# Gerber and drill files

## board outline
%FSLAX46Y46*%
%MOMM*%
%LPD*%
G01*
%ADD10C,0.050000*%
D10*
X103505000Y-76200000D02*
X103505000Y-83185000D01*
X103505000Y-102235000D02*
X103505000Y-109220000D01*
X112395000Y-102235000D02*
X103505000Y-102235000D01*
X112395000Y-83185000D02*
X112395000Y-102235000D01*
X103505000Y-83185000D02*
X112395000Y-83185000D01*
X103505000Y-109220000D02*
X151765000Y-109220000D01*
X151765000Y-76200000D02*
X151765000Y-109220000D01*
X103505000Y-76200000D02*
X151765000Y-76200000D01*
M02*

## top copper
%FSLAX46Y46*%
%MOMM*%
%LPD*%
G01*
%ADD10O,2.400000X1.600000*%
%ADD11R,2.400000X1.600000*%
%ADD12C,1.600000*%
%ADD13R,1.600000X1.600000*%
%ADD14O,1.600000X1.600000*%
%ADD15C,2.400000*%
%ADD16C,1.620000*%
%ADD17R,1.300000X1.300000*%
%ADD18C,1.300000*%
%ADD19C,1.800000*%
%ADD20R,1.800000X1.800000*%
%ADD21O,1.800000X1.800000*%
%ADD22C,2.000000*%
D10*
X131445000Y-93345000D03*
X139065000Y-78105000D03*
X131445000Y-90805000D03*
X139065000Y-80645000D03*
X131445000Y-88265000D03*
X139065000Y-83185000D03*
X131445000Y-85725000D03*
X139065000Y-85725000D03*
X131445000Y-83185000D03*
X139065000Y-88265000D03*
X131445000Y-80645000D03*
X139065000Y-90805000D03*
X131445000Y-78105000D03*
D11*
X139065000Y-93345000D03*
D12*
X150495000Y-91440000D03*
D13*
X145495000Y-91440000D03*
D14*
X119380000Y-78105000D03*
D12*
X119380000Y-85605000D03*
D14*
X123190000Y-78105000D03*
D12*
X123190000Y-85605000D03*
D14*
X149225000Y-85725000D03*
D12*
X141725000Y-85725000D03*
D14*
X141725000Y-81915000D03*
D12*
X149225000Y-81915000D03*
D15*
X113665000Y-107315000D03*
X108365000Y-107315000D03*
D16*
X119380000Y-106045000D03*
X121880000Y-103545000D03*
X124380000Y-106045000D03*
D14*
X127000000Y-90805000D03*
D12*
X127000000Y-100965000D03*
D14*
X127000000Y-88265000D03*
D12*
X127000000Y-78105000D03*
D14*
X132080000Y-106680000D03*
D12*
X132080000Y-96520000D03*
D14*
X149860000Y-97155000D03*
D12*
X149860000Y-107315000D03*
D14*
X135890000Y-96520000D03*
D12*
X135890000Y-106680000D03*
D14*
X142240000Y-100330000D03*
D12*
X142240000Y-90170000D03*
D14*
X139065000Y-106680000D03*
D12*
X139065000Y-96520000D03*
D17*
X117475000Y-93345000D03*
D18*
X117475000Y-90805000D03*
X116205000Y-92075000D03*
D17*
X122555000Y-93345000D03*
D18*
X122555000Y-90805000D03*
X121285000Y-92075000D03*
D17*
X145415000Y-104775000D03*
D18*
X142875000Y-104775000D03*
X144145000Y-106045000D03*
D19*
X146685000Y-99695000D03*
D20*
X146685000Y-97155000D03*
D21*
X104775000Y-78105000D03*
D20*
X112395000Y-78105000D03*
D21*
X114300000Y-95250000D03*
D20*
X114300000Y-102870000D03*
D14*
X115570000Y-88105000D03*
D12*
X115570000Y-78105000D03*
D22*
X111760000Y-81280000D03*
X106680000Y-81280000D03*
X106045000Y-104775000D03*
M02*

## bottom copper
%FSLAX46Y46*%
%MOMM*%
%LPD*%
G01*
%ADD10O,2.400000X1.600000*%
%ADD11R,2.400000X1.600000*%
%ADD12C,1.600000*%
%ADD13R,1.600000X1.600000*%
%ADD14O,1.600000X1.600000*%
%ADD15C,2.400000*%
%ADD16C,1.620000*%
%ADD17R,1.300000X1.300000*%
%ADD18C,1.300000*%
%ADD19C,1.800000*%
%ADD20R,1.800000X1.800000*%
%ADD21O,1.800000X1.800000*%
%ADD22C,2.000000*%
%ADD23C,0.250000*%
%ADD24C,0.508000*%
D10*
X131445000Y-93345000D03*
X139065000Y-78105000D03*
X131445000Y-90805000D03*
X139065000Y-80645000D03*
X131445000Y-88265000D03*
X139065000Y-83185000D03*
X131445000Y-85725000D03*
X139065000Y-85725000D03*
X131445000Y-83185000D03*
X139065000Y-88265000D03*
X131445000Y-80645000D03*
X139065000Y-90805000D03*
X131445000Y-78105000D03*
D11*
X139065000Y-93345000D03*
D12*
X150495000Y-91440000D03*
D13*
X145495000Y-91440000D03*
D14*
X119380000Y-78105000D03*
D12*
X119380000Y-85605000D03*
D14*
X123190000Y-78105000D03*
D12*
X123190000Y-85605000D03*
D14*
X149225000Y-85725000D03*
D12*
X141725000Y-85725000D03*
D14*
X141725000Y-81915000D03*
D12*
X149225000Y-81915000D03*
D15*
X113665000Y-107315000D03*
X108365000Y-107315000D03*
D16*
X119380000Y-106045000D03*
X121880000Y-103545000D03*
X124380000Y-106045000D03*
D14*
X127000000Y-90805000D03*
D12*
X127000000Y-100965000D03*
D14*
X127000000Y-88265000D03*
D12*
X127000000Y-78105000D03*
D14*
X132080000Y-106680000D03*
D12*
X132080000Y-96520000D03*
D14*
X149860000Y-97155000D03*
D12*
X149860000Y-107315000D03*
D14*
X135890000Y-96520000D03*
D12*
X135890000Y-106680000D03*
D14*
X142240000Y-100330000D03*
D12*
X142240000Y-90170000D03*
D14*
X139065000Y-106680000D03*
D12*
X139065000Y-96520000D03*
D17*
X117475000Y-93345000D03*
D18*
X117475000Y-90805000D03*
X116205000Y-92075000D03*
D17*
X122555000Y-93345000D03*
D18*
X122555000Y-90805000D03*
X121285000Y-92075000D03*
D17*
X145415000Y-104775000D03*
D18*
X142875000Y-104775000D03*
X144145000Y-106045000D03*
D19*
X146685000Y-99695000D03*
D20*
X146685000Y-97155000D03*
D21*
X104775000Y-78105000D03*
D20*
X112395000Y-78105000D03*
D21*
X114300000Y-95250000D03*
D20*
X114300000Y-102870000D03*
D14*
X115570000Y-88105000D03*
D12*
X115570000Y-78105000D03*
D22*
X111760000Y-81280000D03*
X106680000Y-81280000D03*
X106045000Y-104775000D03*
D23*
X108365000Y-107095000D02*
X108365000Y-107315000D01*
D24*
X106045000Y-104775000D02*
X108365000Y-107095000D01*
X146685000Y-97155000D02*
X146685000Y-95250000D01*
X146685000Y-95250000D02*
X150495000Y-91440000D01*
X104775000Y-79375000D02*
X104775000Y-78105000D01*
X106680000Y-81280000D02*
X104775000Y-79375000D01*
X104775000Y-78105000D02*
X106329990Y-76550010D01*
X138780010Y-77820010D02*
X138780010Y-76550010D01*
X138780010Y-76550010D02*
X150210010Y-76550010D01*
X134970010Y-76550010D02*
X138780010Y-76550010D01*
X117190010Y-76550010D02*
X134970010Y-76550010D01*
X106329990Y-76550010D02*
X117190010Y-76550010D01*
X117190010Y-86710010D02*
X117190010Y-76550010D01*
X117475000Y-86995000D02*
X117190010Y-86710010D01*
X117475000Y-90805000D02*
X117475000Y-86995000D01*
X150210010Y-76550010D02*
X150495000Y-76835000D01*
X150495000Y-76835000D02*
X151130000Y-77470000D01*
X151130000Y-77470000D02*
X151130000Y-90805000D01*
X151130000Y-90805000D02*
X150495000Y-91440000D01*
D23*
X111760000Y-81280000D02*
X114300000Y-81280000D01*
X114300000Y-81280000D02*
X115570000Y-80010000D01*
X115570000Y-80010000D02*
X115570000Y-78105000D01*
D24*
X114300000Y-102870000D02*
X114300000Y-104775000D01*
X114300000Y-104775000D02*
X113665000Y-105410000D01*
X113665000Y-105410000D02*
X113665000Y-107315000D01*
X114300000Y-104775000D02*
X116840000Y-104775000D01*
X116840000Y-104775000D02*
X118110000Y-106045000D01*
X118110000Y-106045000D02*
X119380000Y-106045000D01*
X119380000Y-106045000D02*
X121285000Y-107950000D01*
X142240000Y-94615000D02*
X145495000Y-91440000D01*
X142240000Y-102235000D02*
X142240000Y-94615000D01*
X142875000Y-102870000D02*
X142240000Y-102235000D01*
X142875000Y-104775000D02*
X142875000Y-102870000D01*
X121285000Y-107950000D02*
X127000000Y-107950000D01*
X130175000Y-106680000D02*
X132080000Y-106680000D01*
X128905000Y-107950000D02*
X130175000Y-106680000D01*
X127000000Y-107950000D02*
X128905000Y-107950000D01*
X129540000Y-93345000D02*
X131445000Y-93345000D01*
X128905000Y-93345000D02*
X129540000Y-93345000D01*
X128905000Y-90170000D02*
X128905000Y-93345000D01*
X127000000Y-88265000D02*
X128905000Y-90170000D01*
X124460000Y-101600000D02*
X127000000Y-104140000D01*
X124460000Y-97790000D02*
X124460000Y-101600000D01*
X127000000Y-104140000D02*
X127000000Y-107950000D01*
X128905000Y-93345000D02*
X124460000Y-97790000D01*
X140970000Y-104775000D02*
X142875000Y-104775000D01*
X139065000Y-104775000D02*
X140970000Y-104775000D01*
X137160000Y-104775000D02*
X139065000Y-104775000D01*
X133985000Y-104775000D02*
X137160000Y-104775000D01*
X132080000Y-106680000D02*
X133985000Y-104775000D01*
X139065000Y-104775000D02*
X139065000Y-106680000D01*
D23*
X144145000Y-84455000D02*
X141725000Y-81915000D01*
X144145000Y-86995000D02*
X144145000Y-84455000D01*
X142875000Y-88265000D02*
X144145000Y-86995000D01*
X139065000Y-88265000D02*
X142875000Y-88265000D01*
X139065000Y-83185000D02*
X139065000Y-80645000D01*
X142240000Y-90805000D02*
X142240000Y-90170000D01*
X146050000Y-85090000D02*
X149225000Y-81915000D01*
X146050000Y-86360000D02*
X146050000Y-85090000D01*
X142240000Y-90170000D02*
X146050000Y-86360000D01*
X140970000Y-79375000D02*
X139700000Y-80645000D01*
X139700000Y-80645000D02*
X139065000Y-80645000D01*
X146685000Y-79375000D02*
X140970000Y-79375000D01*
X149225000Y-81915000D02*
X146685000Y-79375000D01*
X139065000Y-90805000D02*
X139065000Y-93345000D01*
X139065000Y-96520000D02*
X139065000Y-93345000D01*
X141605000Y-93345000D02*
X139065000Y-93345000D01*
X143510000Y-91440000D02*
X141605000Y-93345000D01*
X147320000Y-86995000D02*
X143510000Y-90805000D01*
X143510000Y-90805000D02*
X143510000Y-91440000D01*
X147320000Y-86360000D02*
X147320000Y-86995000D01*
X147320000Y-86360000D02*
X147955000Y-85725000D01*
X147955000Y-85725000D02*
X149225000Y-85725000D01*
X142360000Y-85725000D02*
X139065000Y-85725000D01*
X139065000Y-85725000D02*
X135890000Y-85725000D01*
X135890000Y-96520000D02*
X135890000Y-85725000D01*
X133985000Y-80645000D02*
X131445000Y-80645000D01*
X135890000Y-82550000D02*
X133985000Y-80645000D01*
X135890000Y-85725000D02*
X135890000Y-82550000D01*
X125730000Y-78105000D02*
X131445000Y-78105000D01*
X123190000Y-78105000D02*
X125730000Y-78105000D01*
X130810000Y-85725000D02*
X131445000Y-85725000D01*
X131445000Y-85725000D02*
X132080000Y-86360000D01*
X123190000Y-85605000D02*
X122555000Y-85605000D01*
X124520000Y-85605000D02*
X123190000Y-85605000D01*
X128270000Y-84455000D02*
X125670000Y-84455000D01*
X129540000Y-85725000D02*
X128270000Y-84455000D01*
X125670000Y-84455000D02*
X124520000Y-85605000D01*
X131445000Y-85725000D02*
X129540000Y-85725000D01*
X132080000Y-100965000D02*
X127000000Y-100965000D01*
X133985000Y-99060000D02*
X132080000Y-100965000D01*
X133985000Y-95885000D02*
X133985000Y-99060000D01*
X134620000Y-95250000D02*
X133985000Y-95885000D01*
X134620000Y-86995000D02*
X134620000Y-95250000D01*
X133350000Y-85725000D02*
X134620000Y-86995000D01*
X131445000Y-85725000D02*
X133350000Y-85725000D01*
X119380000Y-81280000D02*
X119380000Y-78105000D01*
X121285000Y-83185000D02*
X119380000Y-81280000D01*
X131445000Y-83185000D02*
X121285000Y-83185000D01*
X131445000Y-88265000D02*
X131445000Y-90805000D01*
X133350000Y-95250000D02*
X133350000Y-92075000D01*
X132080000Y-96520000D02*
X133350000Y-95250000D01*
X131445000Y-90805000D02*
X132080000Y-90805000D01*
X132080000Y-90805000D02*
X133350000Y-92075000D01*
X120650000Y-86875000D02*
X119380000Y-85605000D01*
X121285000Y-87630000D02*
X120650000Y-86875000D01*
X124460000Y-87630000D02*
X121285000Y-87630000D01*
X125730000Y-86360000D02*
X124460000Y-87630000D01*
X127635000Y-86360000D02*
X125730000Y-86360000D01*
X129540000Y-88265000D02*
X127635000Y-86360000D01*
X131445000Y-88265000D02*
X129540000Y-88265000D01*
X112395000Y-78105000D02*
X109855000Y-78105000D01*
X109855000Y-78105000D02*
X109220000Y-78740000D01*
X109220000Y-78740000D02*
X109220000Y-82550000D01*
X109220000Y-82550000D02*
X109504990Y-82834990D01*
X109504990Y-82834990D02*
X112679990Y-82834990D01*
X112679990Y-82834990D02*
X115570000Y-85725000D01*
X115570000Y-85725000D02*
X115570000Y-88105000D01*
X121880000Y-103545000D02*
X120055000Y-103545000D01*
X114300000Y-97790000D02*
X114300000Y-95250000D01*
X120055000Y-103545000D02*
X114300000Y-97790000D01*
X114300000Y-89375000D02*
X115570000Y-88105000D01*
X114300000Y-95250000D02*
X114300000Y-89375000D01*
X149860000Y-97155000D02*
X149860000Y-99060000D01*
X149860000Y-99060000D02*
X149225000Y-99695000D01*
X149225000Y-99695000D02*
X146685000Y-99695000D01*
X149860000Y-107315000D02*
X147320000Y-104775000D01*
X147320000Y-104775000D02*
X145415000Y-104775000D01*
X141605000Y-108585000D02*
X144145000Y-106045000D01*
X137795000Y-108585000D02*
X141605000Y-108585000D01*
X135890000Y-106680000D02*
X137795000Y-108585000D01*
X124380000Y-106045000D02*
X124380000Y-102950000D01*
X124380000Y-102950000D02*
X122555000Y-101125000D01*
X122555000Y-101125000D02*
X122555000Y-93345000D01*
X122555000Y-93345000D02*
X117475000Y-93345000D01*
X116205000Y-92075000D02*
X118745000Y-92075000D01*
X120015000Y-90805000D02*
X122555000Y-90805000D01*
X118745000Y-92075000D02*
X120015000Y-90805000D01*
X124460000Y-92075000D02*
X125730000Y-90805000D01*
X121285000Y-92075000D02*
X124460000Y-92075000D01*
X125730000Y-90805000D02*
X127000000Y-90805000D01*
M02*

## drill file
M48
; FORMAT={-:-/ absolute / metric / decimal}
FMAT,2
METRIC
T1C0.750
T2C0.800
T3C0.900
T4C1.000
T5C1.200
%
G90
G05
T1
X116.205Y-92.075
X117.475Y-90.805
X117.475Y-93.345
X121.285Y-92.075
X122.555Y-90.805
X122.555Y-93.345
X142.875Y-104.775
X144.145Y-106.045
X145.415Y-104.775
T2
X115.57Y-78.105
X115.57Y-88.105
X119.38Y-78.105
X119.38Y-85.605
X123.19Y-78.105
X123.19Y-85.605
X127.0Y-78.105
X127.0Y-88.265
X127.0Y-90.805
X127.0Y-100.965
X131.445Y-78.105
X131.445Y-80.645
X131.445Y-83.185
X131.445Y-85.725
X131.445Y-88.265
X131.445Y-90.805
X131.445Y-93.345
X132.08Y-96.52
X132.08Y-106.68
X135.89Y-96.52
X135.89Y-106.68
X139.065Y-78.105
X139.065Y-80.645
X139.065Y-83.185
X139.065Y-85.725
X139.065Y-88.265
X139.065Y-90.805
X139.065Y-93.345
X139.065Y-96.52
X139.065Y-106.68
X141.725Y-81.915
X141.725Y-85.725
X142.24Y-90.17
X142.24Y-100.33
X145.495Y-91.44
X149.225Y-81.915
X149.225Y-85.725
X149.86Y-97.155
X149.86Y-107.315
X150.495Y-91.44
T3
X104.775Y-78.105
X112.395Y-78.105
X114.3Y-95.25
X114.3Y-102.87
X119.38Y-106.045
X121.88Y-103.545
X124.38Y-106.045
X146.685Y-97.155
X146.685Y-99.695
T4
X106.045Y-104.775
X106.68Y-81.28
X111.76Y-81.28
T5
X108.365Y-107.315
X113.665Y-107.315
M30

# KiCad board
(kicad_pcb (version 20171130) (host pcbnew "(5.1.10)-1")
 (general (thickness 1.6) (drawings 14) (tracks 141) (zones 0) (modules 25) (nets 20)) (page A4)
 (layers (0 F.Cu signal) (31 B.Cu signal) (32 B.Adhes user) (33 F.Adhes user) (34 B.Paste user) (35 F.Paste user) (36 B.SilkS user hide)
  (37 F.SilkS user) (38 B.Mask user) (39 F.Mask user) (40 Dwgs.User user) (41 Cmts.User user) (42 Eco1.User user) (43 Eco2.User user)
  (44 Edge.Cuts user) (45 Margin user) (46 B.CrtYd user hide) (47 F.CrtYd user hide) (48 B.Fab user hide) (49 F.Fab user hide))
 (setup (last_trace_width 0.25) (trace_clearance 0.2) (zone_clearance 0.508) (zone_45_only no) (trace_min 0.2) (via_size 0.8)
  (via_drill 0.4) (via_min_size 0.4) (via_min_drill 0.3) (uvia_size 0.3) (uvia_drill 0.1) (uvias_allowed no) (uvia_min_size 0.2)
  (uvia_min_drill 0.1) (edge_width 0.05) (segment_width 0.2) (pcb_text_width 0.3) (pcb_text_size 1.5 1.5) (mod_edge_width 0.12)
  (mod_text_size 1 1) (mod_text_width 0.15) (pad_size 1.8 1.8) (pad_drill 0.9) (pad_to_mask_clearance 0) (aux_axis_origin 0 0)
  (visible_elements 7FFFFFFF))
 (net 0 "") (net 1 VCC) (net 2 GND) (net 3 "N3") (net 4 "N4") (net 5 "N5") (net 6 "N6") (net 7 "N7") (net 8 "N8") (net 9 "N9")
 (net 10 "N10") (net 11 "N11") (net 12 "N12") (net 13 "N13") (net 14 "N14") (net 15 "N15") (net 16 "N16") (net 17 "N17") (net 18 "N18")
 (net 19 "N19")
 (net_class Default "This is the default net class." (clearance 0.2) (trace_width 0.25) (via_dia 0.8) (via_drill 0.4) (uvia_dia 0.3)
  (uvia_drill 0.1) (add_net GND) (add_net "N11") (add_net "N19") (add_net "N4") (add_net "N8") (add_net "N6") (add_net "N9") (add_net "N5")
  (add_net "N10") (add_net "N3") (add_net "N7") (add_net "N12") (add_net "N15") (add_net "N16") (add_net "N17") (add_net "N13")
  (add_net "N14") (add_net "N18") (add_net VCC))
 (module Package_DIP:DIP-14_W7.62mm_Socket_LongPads (layer F.Cu) (at 139.065 93.345 180)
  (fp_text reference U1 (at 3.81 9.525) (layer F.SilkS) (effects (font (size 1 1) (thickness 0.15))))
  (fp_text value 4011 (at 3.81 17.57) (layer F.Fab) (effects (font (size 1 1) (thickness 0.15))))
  (pad 14 thru_hole oval (at 7.62 0 180) (size 2.4 1.6) (drill 0.8) (layers *.Cu *.Mask) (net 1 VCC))
  (pad 7 thru_hole oval (at 0 15.24 180) (size 2.4 1.6) (drill 0.8) (layers *.Cu *.Mask) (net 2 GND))
  (pad 13 thru_hole oval (at 7.62 2.54 180) (size 2.4 1.6) (drill 0.8) (layers *.Cu *.Mask) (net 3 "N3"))
  (pad 6 thru_hole oval (at 0 12.7 180) (size 2.4 1.6) (drill 0.8) (layers *.Cu *.Mask) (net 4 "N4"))
  (pad 12 thru_hole oval (at 7.62 5.08 180) (size 2.4 1.6) (drill 0.8) (layers *.Cu *.Mask) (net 3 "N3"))
  (pad 5 thru_hole oval (at 0 10.16 180) (size 2.4 1.6) (drill 0.8) (layers *.Cu *.Mask) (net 4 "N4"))
  (pad 11 thru_hole oval (at 7.62 7.62 180) (size 2.4 1.6) (drill 0.8) (layers *.Cu *.Mask) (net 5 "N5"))
  (pad 4 thru_hole oval (at 0 7.62 180) (size 2.4 1.6) (drill 0.8) (layers *.Cu *.Mask) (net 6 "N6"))
  (pad 10 thru_hole oval (at 7.62 10.16 180) (size 2.4 1.6) (drill 0.8) (layers *.Cu *.Mask) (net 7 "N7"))
  (pad 3 thru_hole oval (at 0 5.08 180) (size 2.4 1.6) (drill 0.8) (layers *.Cu *.Mask) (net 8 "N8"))
  (pad 9 thru_hole oval (at 7.62 12.7 180) (size 2.4 1.6) (drill 0.8) (layers *.Cu *.Mask) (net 6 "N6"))
  (pad 2 thru_hole oval (at 0 2.54 180) (size 2.4 1.6) (drill 0.8) (layers *.Cu *.Mask) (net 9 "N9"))
  (pad 8 thru_hole oval (at 7.62 15.24 180) (size 2.4 1.6) (drill 0.8) (layers *.Cu *.Mask) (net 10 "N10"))
  (pad 1 thru_hole rect (at 0 0 180) (size 2.4 1.6) (drill 0.8) (layers *.Cu *.Mask) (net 9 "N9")))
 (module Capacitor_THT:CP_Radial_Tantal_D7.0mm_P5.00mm (layer F.Cu) (at 145.495 91.44)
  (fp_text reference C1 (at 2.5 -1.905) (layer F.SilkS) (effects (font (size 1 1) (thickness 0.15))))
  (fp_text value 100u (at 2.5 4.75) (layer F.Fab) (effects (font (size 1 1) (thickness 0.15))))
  (pad 2 thru_hole circle (at 5 0) (size 1.6 1.6) (drill 0.8) (layers *.Cu *.Mask) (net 2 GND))
  (pad 1 thru_hole rect (at 0 0) (size 1.6 1.6) (drill 0.8) (layers *.Cu *.Mask) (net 1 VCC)))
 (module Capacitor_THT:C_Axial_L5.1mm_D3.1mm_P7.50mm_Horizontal (layer F.Cu) (at 119.38 85.605 90)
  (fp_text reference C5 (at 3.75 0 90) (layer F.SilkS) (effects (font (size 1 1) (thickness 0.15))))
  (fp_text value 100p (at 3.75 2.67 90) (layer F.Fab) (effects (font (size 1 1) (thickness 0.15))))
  (pad 2 thru_hole oval (at 7.5 0 90) (size 1.6 1.6) (drill 0.8) (layers *.Cu *.Mask) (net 7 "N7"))
  (pad 1 thru_hole circle (at 0 0 90) (size 1.6 1.6) (drill 0.8) (layers *.Cu *.Mask) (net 3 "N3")))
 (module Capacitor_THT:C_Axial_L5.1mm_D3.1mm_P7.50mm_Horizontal (layer F.Cu) (at 123.19 85.605 90)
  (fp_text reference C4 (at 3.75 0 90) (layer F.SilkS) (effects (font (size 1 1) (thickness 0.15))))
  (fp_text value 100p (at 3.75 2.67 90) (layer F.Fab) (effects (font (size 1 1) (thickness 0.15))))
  (pad 2 thru_hole oval (at 7.5 0 90) (size 1.6 1.6) (drill 0.8) (layers *.Cu *.Mask) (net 10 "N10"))
  (pad 1 thru_hole circle (at 0 0 90) (size 1.6 1.6) (drill 0.8) (layers *.Cu *.Mask) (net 5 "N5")))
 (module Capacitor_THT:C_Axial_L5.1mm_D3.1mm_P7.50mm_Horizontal (layer F.Cu) (at 141.725 85.725)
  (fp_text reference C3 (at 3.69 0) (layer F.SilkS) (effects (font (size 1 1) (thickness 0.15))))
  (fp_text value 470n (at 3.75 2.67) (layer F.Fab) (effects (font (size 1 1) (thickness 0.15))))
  (pad 2 thru_hole oval (at 7.5 0) (size 1.6 1.6) (drill 0.8) (layers *.Cu *.Mask) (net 9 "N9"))
  (pad 1 thru_hole circle (at 0 0) (size 1.6 1.6) (drill 0.8) (layers *.Cu *.Mask) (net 6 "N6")))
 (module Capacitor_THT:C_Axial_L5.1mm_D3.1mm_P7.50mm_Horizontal (layer F.Cu) (at 149.225 81.915 180)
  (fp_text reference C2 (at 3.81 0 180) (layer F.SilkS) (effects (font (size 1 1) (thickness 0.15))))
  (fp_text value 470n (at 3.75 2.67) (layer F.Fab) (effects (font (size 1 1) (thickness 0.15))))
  (pad 2 thru_hole oval (at 7.5 0 180) (size 1.6 1.6) (drill 0.8) (layers *.Cu *.Mask) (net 8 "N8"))
  (pad 1 thru_hole circle (at 0 0 180) (size 1.6 1.6) (drill 0.8) (layers *.Cu *.Mask) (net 4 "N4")))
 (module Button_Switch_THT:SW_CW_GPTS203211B (layer B.Cu) (at 108.365 107.315 270)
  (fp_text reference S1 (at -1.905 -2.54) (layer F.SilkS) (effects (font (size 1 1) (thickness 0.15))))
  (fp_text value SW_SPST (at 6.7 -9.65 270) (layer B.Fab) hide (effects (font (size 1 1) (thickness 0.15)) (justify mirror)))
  (pad 2 thru_hole circle (at 0 -5.3 270) (size 2.4 2.4) (drill 1.2) (layers *.Cu *.Mask) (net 1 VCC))
  (pad 1 thru_hole circle (at 0 0 270) (size 2.4 2.4) (drill 1.2) (layers *.Cu *.Mask) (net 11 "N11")))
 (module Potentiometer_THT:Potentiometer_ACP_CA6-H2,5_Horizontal (layer F.Cu) (at 119.38 106.045 90)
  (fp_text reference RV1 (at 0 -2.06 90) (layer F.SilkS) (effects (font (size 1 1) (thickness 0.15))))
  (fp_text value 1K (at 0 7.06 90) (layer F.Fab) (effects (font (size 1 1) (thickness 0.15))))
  (pad 1 thru_hole circle (at 0 0 90) (size 1.62 1.62) (drill 0.9) (layers *.Cu *.Mask) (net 1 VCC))
  (pad 2 thru_hole circle (at 2.5 2.5 90) (size 1.62 1.62) (drill 0.9) (layers *.Cu *.Mask) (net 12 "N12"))
  (pad 3 thru_hole circle (at 0 5 90) (size 1.62 1.62) (drill 0.9) (layers *.Cu *.Mask) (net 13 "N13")))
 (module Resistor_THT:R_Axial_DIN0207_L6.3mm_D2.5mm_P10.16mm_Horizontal (layer F.Cu) (at 127 100.965 90)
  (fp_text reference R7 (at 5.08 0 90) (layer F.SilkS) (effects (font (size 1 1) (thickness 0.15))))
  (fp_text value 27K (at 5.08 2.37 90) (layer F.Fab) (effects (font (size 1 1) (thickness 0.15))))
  (pad 2 thru_hole oval (at 10.16 0 90) (size 1.6 1.6) (drill 0.8) (layers *.Cu *.Mask) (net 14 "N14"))
  (pad 1 thru_hole circle (at 0 0 90) (size 1.6 1.6) (drill 0.8) (layers *.Cu *.Mask) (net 5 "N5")))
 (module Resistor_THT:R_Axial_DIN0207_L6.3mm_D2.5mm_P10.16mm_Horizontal (layer F.Cu) (at 127 78.105 270)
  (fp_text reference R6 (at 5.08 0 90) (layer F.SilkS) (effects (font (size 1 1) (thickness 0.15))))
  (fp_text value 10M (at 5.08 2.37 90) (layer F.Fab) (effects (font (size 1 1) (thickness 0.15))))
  (pad 2 thru_hole oval (at 10.16 0 270) (size 1.6 1.6) (drill 0.8) (layers *.Cu *.Mask) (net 1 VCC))
  (pad 1 thru_hole circle (at 0 0 270) (size 1.6 1.6) (drill 0.8) (layers *.Cu *.Mask) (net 10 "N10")))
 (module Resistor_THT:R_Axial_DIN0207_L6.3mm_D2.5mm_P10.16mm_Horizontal (layer F.Cu) (at 132.08 96.52 270)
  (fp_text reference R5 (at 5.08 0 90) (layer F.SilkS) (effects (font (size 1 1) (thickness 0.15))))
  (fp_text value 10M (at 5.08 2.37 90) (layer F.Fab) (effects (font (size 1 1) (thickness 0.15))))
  (pad 2 thru_hole oval (at 10.16 0 270) (size 1.6 1.6) (drill 0.8) (layers *.Cu *.Mask) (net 1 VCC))
  (pad 1 thru_hole circle (at 0 0 270) (size 1.6 1.6) (drill 0.8) (layers *.Cu *.Mask) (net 3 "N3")))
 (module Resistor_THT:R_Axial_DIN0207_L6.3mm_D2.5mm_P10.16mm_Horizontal (layer F.Cu) (at 149.86 107.315 90)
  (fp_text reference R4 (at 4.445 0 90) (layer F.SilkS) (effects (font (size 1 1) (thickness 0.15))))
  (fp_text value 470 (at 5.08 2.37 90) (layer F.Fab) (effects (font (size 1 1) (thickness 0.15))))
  (pad 2 thru_hole oval (at 10.16 0 90) (size 1.6 1.6) (drill 0.8) (layers *.Cu *.Mask) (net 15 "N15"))
  (pad 1 thru_hole circle (at 0 0 90) (size 1.6 1.6) (drill 0.8) (layers *.Cu *.Mask) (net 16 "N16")))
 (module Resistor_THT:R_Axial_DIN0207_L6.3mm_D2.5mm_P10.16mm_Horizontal (layer F.Cu) (at 135.89 106.68 90)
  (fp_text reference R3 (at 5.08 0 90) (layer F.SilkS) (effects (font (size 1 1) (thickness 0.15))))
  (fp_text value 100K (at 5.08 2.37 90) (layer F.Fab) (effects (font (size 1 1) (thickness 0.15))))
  (pad 2 thru_hole oval (at 10.16 0 90) (size 1.6 1.6) (drill 0.8) (layers *.Cu *.Mask) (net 6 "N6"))
  (pad 1 thru_hole circle (at 0 0 90) (size 1.6 1.6) (drill 0.8) (layers *.Cu *.Mask) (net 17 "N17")))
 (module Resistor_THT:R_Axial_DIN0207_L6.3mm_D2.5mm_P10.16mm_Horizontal (layer F.Cu) (at 142.24 90.17 270)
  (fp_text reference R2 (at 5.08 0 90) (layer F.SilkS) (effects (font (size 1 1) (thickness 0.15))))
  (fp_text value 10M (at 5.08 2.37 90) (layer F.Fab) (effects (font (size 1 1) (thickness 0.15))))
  (pad 2 thru_hole oval (at 10.16 0 270) (size 1.6 1.6) (drill 0.8) (layers *.Cu *.Mask) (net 1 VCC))
  (pad 1 thru_hole circle (at 0 0 270) (size 1.6 1.6) (drill 0.8) (layers *.Cu *.Mask) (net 4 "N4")))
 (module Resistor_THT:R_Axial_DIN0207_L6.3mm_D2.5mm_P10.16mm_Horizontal (layer F.Cu) (at 139.065 96.52 270)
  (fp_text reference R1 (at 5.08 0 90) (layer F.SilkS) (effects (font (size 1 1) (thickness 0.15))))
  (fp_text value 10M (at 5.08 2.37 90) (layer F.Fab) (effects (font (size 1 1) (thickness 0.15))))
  (pad 2 thru_hole oval (at 10.16 0 270) (size 1.6 1.6) (drill 0.8) (layers *.Cu *.Mask) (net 1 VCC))
  (pad 1 thru_hole circle (at 0 0 270) (size 1.6 1.6) (drill 0.8) (layers *.Cu *.Mask) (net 9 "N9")))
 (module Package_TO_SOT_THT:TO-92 (layer F.Cu) (at 117.475 93.345 90)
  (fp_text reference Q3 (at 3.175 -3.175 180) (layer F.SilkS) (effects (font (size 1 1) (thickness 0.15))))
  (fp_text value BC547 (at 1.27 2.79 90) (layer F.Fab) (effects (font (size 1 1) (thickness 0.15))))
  (pad 1 thru_hole rect (at 0 0 90) (size 1.3 1.3) (drill 0.75) (layers *.Cu *.Mask) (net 13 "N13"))
  (pad 3 thru_hole circle (at 2.54 0 90) (size 1.3 1.3) (drill 0.75) (layers *.Cu *.Mask) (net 2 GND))
  (pad 2 thru_hole circle (at 1.27 -1.27 90) (size 1.3 1.3) (drill 0.75) (layers *.Cu *.Mask) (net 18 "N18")))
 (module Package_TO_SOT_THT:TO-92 (layer F.Cu) (at 122.555 93.345 90)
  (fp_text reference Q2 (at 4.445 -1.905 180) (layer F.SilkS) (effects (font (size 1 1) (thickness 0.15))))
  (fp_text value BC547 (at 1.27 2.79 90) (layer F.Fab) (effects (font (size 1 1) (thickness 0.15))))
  (pad 1 thru_hole rect (at 0 0 90) (size 1.3 1.3) (drill 0.75) (layers *.Cu *.Mask) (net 13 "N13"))
  (pad 3 thru_hole circle (at 2.54 0 90) (size 1.3 1.3) (drill 0.75) (layers *.Cu *.Mask) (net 18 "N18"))
  (pad 2 thru_hole circle (at 1.27 -1.27 90) (size 1.3 1.3) (drill 0.75) (layers *.Cu *.Mask) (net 14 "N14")))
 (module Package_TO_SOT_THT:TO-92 (layer F.Cu) (at 145.415 104.775 180)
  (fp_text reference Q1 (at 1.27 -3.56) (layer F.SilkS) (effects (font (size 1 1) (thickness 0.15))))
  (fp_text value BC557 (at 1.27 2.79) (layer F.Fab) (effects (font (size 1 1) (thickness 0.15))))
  (pad 1 thru_hole rect (at 0 0 180) (size 1.3 1.3) (drill 0.75) (layers *.Cu *.Mask) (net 16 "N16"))
  (pad 3 thru_hole circle (at 2.54 0 180) (size 1.3 1.3) (drill 0.75) (layers *.Cu *.Mask) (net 1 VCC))
  (pad 2 thru_hole circle (at 1.27 -1.27 180) (size 1.3 1.3) (drill 0.75) (layers *.Cu *.Mask) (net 17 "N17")))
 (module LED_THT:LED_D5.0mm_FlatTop (layer F.Cu) (at 146.685 97.155 270)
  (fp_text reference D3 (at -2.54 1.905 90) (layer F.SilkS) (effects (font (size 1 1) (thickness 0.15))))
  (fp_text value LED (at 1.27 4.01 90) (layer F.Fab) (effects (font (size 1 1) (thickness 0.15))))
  (pad 2 thru_hole circle (at 2.54 0 270) (size 1.8 1.8) (drill 0.9) (layers *.Cu *.Mask) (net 15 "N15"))
  (pad 1 thru_hole rect (at 0 0 270) (size 1.8 1.8) (drill 0.9) (layers *.Cu *.Mask) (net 2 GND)))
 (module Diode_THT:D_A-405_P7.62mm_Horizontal (layer F.Cu) (at 112.395 78.105 180)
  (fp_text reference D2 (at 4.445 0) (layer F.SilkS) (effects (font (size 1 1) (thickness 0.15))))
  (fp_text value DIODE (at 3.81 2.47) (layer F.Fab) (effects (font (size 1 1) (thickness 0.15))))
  (pad 1 thru_hole oval (at 7.62 0 180) (size 1.8 1.8) (drill 0.9) (layers *.Cu *.Mask) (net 2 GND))
  (pad 2 thru_hole rect (at 0 0 180) (size 1.8 1.8) (drill 0.9) (layers *.Cu *.Mask) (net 12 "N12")))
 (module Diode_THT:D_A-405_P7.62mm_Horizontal (layer F.Cu) (at 114.3 102.87 90)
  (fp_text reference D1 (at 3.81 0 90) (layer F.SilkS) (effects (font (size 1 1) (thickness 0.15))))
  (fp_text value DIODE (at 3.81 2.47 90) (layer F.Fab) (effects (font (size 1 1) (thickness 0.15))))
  (pad 1 thru_hole oval (at 7.62 0 90) (size 1.8 1.8) (drill 0.9) (layers *.Cu *.Mask) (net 12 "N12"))
  (pad 2 thru_hole rect (at 0 0 90) (size 1.8 1.8) (drill 0.9) (layers *.Cu *.Mask) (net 1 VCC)))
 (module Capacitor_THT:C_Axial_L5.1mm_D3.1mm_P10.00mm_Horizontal (layer F.Cu) (at 115.57 78.105 270)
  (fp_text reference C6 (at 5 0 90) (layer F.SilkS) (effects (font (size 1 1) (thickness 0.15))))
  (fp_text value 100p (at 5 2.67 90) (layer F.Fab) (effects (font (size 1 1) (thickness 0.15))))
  (pad 2 thru_hole oval (at 10 0 270) (size 1.6 1.6) (drill 0.8) (layers *.Cu *.Mask) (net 12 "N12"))
  (pad 1 thru_hole circle (at 0 0 270) (size 1.6 1.6) (drill 0.8) (layers *.Cu *.Mask) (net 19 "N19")))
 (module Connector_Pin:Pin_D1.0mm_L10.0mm (layer F.Cu) (at 111.76 81.28)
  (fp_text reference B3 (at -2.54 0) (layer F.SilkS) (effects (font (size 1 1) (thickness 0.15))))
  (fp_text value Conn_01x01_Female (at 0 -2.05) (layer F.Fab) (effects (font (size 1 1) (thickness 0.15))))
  (pad 1 thru_hole circle (at 0 0) (size 2 2) (drill 1) (layers *.Cu *.Mask) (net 19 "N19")))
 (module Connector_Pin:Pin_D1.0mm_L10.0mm (layer F.Cu) (at 106.68 81.28)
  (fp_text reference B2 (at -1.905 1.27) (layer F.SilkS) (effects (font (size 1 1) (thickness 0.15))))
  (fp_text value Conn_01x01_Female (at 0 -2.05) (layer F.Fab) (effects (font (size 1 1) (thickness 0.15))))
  (pad 1 thru_hole circle (at 0 0) (size 2 2) (drill 1) (layers *.Cu *.Mask) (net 2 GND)))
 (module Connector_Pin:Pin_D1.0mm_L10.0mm (layer F.Cu) (at 106.045 104.775)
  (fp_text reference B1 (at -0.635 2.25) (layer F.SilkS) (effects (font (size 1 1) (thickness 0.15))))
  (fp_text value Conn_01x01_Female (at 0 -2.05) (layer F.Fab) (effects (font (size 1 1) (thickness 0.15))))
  (pad 1 thru_hole circle (at 0 0) (size 2 2) (drill 1) (layers *.Cu *.Mask) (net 11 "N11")))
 (gr_line (start 103.505 76.2) (end 103.505 83.185) (layer Edge.Cuts) (width 0.05))
 (gr_line (start 103.505 102.235) (end 103.505 109.22) (layer Edge.Cuts) (width 0.05))
 (gr_line (start 112.395 102.235) (end 103.505 102.235) (layer Edge.Cuts) (width 0.05))
 (gr_line (start 112.395 83.185) (end 112.395 102.235) (layer Edge.Cuts) (width 0.05))
 (gr_line (start 103.505 83.185) (end 112.395 83.185) (layer Edge.Cuts) (width 0.05))
 (gr_line (start 103.505 109.22) (end 151.765 109.22) (layer Edge.Cuts) (width 0.05))
 (gr_line (start 151.765 76.2) (end 151.765 109.22) (layer Edge.Cuts) (width 0.05))
 (gr_line (start 103.505 76.2) (end 151.765 76.2) (layer Edge.Cuts) (width 0.05))
 (segment (start 108.365 107.095) (end 108.365 107.315) (width 0.25) (layer B.Cu) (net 11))
 (segment (start 106.045 104.775) (end 108.365 107.095) (width 0.508) (layer B.Cu) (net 11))
 (segment (start 146.685 97.155) (end 146.685 95.25) (width 0.508) (layer B.Cu) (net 2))
 (segment (start 146.685 95.25) (end 150.495 91.44) (width 0.508) (layer B.Cu) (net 2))
 (segment (start 104.775 79.375) (end 104.775 78.105) (width 0.508) (layer B.Cu) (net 2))
 (segment (start 106.68 81.28) (end 104.775 79.375) (width 0.508) (layer B.Cu) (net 2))
 (segment (start 104.775 78.105) (end 106.32999 76.55001) (width 0.508) (layer B.Cu) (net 2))
 (segment (start 138.78001 77.82001) (end 138.78001 76.55001) (width 0.508) (layer B.Cu) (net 2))
 (segment (start 138.78001 76.55001) (end 150.21001 76.55001) (width 0.508) (layer B.Cu) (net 2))
 (segment (start 134.97001 76.55001) (end 138.78001 76.55001) (width 0.508) (layer B.Cu) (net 2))
 (segment (start 117.19001 76.55001) (end 134.97001 76.55001) (width 0.508) (layer B.Cu) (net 2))
 (segment (start 106.32999 76.55001) (end 117.19001 76.55001) (width 0.508) (layer B.Cu) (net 2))
 (segment (start 117.19001 86.71001) (end 117.19001 76.55001) (width 0.508) (layer B.Cu) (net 2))
 (segment (start 117.475 86.995) (end 117.19001 86.71001) (width 0.508) (layer B.Cu) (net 2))
 (segment (start 117.475 90.805) (end 117.475 86.995) (width 0.508) (layer B.Cu) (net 2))
 (segment (start 150.21001 76.55001) (end 150.495 76.835) (width 0.508) (layer B.Cu) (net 2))
 (segment (start 150.495 76.835) (end 151.13 77.47) (width 0.508) (layer B.Cu) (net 2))
 (segment (start 151.13 77.47) (end 151.13 90.805) (width 0.508) (layer B.Cu) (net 2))
 (segment (start 151.13 90.805) (end 150.495 91.44) (width 0.508) (layer B.Cu) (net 2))
 (segment (start 111.76 81.28) (end 114.3 81.28) (width 0.25) (layer B.Cu) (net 19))
 (segment (start 114.3 81.28) (end 115.57 80.01) (width 0.25) (layer B.Cu) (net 19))
 (segment (start 115.57 80.01) (end 115.57 78.105) (width 0.25) (layer B.Cu) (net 19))
 (segment (start 114.3 102.87) (end 114.3 104.775) (width 0.508) (layer B.Cu) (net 1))
 (segment (start 114.3 104.775) (end 113.665 105.41) (width 0.508) (layer B.Cu) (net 1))
 (segment (start 113.665 105.41) (end 113.665 107.315) (width 0.508) (layer B.Cu) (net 1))
 (segment (start 114.3 104.775) (end 116.84 104.775) (width 0.508) (layer B.Cu) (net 1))
 (segment (start 116.84 104.775) (end 118.11 106.045) (width 0.508) (layer B.Cu) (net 1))
 (segment (start 118.11 106.045) (end 119.38 106.045) (width 0.508) (layer B.Cu) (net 1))
 (segment (start 119.38 106.045) (end 121.285 107.95) (width 0.508) (layer B.Cu) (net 1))
 (segment (start 142.24 94.615) (end 145.495 91.44) (width 0.508) (layer B.Cu) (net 1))
 (segment (start 142.24 102.235) (end 142.24 94.615) (width 0.508) (layer B.Cu) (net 1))
 (segment (start 142.875 102.87) (end 142.24 102.235) (width 0.508) (layer B.Cu) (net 1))
 (segment (start 142.875 104.775) (end 142.875 102.87) (width 0.508) (layer B.Cu) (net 1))
 (segment (start 121.285 107.95) (end 127 107.95) (width 0.508) (layer B.Cu) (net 1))
 (segment (start 130.175 106.68) (end 132.08 106.68) (width 0.508) (layer B.Cu) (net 1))
 (segment (start 128.905 107.95) (end 130.175 106.68) (width 0.508) (layer B.Cu) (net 1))
 (segment (start 127 107.95) (end 128.905 107.95) (width 0.508) (layer B.Cu) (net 1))
 (segment (start 129.54 93.345) (end 131.445 93.345) (width 0.508) (layer B.Cu) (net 1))
 (segment (start 128.905 93.345) (end 129.54 93.345) (width 0.508) (layer B.Cu) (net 1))
 (segment (start 128.905 90.17) (end 128.905 93.345) (width 0.508) (layer B.Cu) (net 1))
 (segment (start 127 88.265) (end 128.905 90.17) (width 0.508) (layer B.Cu) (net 1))
 (segment (start 124.46 101.6) (end 127 104.14) (width 0.508) (layer B.Cu) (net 1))
 (segment (start 124.46 97.79) (end 124.46 101.6) (width 0.508) (layer B.Cu) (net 1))
 (segment (start 127 104.14) (end 127 107.95) (width 0.508) (layer B.Cu) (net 1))
 (segment (start 128.905 93.345) (end 124.46 97.79) (width 0.508) (layer B.Cu) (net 1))
 (segment (start 140.97 104.775) (end 142.875 104.775) (width 0.508) (layer B.Cu) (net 1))
 (segment (start 139.065 104.775) (end 140.97 104.775) (width 0.508) (layer B.Cu) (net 1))
 (segment (start 137.16 104.775) (end 139.065 104.775) (width 0.508) (layer B.Cu) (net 1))
 (segment (start 133.985 104.775) (end 137.16 104.775) (width 0.508) (layer B.Cu) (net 1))
 (segment (start 132.08 106.68) (end 133.985 104.775) (width 0.508) (layer B.Cu) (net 1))
 (segment (start 139.065 104.775) (end 139.065 106.68) (width 0.508) (layer B.Cu) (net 1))
 (segment (start 144.145 84.455) (end 141.725 81.915) (width 0.25) (layer B.Cu) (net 8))
 (segment (start 144.145 86.995) (end 144.145 84.455) (width 0.25) (layer B.Cu) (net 8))
 (segment (start 142.875 88.265) (end 144.145 86.995) (width 0.25) (layer B.Cu) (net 8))
 (segment (start 139.065 88.265) (end 142.875 88.265) (width 0.25) (layer B.Cu) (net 8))
 (segment (start 139.065 83.185) (end 139.065 80.645) (width 0.25) (layer B.Cu) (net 4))
 (segment (start 142.24 90.805) (end 142.24 90.17) (width 0.25) (layer B.Cu) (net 4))
 (segment (start 146.05 85.09) (end 149.225 81.915) (width 0.25) (layer B.Cu) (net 4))
 (segment (start 146.05 86.36) (end 146.05 85.09) (width 0.25) (layer B.Cu) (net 4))
 (segment (start 142.24 90.17) (end 146.05 86.36) (width 0.25) (layer B.Cu) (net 4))
 (segment (start 140.97 79.375) (end 139.7 80.645) (width 0.25) (layer B.Cu) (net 4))
 (segment (start 139.7 80.645) (end 139.065 80.645) (width 0.25) (layer B.Cu) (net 4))
 (segment (start 146.685 79.375) (end 140.97 79.375) (width 0.25) (layer B.Cu) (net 4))
 (segment (start 149.225 81.915) (end 146.685 79.375) (width 0.25) (layer B.Cu) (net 4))
 (segment (start 139.065 90.805) (end 139.065 93.345) (width 0.25) (layer B.Cu) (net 9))
 (segment (start 139.065 96.52) (end 139.065 93.345) (width 0.25) (layer B.Cu) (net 9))
 (segment (start 141.605 93.345) (end 139.065 93.345) (width 0.25) (layer B.Cu) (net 9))
 (segment (start 143.51 91.44) (end 141.605 93.345) (width 0.25) (layer B.Cu) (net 9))
 (segment (start 147.32 86.995) (end 143.51 90.805) (width 0.25) (layer B.Cu) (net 9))
 (segment (start 143.51 90.805) (end 143.51 91.44) (width 0.25) (layer B.Cu) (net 9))
 (segment (start 147.32 86.36) (end 147.32 86.995) (width 0.25) (layer B.Cu) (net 9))
 (segment (start 147.32 86.36) (end 147.955 85.725) (width 0.25) (layer B.Cu) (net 9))
 (segment (start 147.955 85.725) (end 149.225 85.725) (width 0.25) (layer B.Cu) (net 9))
 (segment (start 142.36 85.725) (end 139.065 85.725) (width 0.25) (layer B.Cu) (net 6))
 (segment (start 139.065 85.725) (end 135.89 85.725) (width 0.25) (layer B.Cu) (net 6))
 (segment (start 135.89 96.52) (end 135.89 85.725) (width 0.25) (layer B.Cu) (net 6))
 (segment (start 133.985 80.645) (end 131.445 80.645) (width 0.25) (layer B.Cu) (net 6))
 (segment (start 135.89 82.55) (end 133.985 80.645) (width 0.25) (layer B.Cu) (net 6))
 (segment (start 135.89 85.725) (end 135.89 82.55) (width 0.25) (layer B.Cu) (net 6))
 (segment (start 125.73 78.105) (end 131.445 78.105) (width 0.25) (layer B.Cu) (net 10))
 (segment (start 123.19 78.105) (end 125.73 78.105) (width 0.25) (layer B.Cu) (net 10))
 (segment (start 130.81 85.725) (end 131.445 85.725) (width 0.25) (layer B.Cu) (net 5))
 (segment (start 131.445 85.725) (end 132.08 86.36) (width 0.25) (layer B.Cu) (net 5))
 (segment (start 123.19 85.605) (end 122.555 85.605) (width 0.25) (layer B.Cu) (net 5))
 (segment (start 124.52 85.605) (end 123.19 85.605) (width 0.25) (layer B.Cu) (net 5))
 (segment (start 128.27 84.455) (end 125.67 84.455) (width 0.25) (layer B.Cu) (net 5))
 (segment (start 129.54 85.725) (end 128.27 84.455) (width 0.25) (layer B.Cu) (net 5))
 (segment (start 125.67 84.455) (end 124.52 85.605) (width 0.25) (layer B.Cu) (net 5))
 (segment (start 131.445 85.725) (end 129.54 85.725) (width 0.25) (layer B.Cu) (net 5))
 (segment (start 132.08 100.965) (end 127 100.965) (width 0.25) (layer B.Cu) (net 5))
 (segment (start 133.985 99.06) (end 132.08 100.965) (width 0.25) (layer B.Cu) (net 5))
 (segment (start 133.985 95.885) (end 133.985 99.06) (width 0.25) (layer B.Cu) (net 5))
 (segment (start 134.62 95.25) (end 133.985 95.885) (width 0.25) (layer B.Cu) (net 5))
 (segment (start 134.62 86.995) (end 134.62 95.25) (width 0.25) (layer B.Cu) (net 5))
 (segment (start 133.35 85.725) (end 134.62 86.995) (width 0.25) (layer B.Cu) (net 5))
 (segment (start 131.445 85.725) (end 133.35 85.725) (width 0.25) (layer B.Cu) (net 5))
 (segment (start 119.38 81.28) (end 119.38 78.105) (width 0.25) (layer B.Cu) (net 7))
 (segment (start 121.285 83.185) (end 119.38 81.28) (width 0.25) (layer B.Cu) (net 7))
 (segment (start 131.445 83.185) (end 121.285 83.185) (width 0.25) (layer B.Cu) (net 7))
 (segment (start 131.445 88.265) (end 131.445 90.805) (width 0.25) (layer B.Cu) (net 3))
 (segment (start 133.35 95.25) (end 133.35 92.075) (width 0.25) (layer B.Cu) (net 3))
 (segment (start 132.08 96.52) (end 133.35 95.25) (width 0.25) (layer B.Cu) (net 3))
 (segment (start 131.445 90.805) (end 132.08 90.805) (width 0.25) (layer B.Cu) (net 3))
 (segment (start 132.08 90.805) (end 133.35 92.075) (width 0.25) (layer B.Cu) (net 3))
 (segment (start 120.65 86.875) (end 119.38 85.605) (width 0.25) (layer B.Cu) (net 3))
 (segment (start 121.285 87.63) (end 120.65 86.875) (width 0.25) (layer B.Cu) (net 3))
 (segment (start 124.46 87.63) (end 121.285 87.63) (width 0.25) (layer B.Cu) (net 3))
 (segment (start 125.73 86.36) (end 124.46 87.63) (width 0.25) (layer B.Cu) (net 3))
 (segment (start 127.635 86.36) (end 125.73 86.36) (width 0.25) (layer B.Cu) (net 3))
 (segment (start 129.54 88.265) (end 127.635 86.36) (width 0.25) (layer B.Cu) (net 3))
 (segment (start 131.445 88.265) (end 129.54 88.265) (width 0.25) (layer B.Cu) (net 3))
 (segment (start 112.395 78.105) (end 109.855 78.105) (width 0.25) (layer B.Cu) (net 12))
 (segment (start 109.855 78.105) (end 109.22 78.74) (width 0.25) (layer B.Cu) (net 12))
 (segment (start 109.22 78.74) (end 109.22 82.55) (width 0.25) (layer B.Cu) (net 12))
 (segment (start 109.22 82.55) (end 109.50499 82.83499) (width 0.25) (layer B.Cu) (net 12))
 (segment (start 109.50499 82.83499) (end 112.67999 82.83499) (width 0.25) (layer B.Cu) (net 12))
 (segment (start 112.67999 82.83499) (end 115.57 85.725) (width 0.25) (layer B.Cu) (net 12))
 (segment (start 115.57 85.725) (end 115.57 88.105) (width 0.25) (layer B.Cu) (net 12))
 (segment (start 121.88 103.545) (end 120.055 103.545) (width 0.25) (layer B.Cu) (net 12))
 (segment (start 114.3 97.79) (end 114.3 95.25) (width 0.25) (layer B.Cu) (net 12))
 (segment (start 120.055 103.545) (end 114.3 97.79) (width 0.25) (layer B.Cu) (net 12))
 (segment (start 114.3 89.375) (end 115.57 88.105) (width 0.25) (layer B.Cu) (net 12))
 (segment (start 114.3 95.25) (end 114.3 89.375) (width 0.25) (layer B.Cu) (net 12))
 (segment (start 149.86 97.155) (end 149.86 99.06) (width 0.25) (layer B.Cu) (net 15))
 (segment (start 149.86 99.06) (end 149.225 99.695) (width 0.25) (layer B.Cu) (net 15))
 (segment (start 149.225 99.695) (end 146.685 99.695) (width 0.25) (layer B.Cu) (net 15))
 (segment (start 149.86 107.315) (end 147.32 104.775) (width 0.25) (layer B.Cu) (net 16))
 (segment (start 147.32 104.775) (end 145.415 104.775) (width 0.25) (layer B.Cu) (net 16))
 (segment (start 141.605 108.585) (end 144.145 106.045) (width 0.25) (layer B.Cu) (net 17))
 (segment (start 137.795 108.585) (end 141.605 108.585) (width 0.25) (layer B.Cu) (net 17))
 (segment (start 135.89 106.68) (end 137.795 108.585) (width 0.25) (layer B.Cu) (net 17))
 (segment (start 124.38 106.045) (end 124.38 102.95) (width 0.25) (layer B.Cu) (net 13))
 (segment (start 124.38 102.95) (end 122.555 101.125) (width 0.25) (layer B.Cu) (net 13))
 (segment (start 122.555 101.125) (end 122.555 93.345) (width 0.25) (layer B.Cu) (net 13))
 (segment (start 122.555 93.345) (end 117.475 93.345) (width 0.25) (layer B.Cu) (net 13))
 (segment (start 116.205 92.075) (end 118.745 92.075) (width 0.25) (layer B.Cu) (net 18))
 (segment (start 120.015 90.805) (end 122.555 90.805) (width 0.25) (layer B.Cu) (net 18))
 (segment (start 118.745 92.075) (end 120.015 90.805) (width 0.25) (layer B.Cu) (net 18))
 (segment (start 124.46 92.075) (end 125.73 90.805) (width 0.25) (layer B.Cu) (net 14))
 (segment (start 121.285 92.075) (end 124.46 92.075) (width 0.25) (layer B.Cu) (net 14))
 (segment (start 125.73 90.805) (end 127 90.805) (width 0.25) (layer B.Cu) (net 14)))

